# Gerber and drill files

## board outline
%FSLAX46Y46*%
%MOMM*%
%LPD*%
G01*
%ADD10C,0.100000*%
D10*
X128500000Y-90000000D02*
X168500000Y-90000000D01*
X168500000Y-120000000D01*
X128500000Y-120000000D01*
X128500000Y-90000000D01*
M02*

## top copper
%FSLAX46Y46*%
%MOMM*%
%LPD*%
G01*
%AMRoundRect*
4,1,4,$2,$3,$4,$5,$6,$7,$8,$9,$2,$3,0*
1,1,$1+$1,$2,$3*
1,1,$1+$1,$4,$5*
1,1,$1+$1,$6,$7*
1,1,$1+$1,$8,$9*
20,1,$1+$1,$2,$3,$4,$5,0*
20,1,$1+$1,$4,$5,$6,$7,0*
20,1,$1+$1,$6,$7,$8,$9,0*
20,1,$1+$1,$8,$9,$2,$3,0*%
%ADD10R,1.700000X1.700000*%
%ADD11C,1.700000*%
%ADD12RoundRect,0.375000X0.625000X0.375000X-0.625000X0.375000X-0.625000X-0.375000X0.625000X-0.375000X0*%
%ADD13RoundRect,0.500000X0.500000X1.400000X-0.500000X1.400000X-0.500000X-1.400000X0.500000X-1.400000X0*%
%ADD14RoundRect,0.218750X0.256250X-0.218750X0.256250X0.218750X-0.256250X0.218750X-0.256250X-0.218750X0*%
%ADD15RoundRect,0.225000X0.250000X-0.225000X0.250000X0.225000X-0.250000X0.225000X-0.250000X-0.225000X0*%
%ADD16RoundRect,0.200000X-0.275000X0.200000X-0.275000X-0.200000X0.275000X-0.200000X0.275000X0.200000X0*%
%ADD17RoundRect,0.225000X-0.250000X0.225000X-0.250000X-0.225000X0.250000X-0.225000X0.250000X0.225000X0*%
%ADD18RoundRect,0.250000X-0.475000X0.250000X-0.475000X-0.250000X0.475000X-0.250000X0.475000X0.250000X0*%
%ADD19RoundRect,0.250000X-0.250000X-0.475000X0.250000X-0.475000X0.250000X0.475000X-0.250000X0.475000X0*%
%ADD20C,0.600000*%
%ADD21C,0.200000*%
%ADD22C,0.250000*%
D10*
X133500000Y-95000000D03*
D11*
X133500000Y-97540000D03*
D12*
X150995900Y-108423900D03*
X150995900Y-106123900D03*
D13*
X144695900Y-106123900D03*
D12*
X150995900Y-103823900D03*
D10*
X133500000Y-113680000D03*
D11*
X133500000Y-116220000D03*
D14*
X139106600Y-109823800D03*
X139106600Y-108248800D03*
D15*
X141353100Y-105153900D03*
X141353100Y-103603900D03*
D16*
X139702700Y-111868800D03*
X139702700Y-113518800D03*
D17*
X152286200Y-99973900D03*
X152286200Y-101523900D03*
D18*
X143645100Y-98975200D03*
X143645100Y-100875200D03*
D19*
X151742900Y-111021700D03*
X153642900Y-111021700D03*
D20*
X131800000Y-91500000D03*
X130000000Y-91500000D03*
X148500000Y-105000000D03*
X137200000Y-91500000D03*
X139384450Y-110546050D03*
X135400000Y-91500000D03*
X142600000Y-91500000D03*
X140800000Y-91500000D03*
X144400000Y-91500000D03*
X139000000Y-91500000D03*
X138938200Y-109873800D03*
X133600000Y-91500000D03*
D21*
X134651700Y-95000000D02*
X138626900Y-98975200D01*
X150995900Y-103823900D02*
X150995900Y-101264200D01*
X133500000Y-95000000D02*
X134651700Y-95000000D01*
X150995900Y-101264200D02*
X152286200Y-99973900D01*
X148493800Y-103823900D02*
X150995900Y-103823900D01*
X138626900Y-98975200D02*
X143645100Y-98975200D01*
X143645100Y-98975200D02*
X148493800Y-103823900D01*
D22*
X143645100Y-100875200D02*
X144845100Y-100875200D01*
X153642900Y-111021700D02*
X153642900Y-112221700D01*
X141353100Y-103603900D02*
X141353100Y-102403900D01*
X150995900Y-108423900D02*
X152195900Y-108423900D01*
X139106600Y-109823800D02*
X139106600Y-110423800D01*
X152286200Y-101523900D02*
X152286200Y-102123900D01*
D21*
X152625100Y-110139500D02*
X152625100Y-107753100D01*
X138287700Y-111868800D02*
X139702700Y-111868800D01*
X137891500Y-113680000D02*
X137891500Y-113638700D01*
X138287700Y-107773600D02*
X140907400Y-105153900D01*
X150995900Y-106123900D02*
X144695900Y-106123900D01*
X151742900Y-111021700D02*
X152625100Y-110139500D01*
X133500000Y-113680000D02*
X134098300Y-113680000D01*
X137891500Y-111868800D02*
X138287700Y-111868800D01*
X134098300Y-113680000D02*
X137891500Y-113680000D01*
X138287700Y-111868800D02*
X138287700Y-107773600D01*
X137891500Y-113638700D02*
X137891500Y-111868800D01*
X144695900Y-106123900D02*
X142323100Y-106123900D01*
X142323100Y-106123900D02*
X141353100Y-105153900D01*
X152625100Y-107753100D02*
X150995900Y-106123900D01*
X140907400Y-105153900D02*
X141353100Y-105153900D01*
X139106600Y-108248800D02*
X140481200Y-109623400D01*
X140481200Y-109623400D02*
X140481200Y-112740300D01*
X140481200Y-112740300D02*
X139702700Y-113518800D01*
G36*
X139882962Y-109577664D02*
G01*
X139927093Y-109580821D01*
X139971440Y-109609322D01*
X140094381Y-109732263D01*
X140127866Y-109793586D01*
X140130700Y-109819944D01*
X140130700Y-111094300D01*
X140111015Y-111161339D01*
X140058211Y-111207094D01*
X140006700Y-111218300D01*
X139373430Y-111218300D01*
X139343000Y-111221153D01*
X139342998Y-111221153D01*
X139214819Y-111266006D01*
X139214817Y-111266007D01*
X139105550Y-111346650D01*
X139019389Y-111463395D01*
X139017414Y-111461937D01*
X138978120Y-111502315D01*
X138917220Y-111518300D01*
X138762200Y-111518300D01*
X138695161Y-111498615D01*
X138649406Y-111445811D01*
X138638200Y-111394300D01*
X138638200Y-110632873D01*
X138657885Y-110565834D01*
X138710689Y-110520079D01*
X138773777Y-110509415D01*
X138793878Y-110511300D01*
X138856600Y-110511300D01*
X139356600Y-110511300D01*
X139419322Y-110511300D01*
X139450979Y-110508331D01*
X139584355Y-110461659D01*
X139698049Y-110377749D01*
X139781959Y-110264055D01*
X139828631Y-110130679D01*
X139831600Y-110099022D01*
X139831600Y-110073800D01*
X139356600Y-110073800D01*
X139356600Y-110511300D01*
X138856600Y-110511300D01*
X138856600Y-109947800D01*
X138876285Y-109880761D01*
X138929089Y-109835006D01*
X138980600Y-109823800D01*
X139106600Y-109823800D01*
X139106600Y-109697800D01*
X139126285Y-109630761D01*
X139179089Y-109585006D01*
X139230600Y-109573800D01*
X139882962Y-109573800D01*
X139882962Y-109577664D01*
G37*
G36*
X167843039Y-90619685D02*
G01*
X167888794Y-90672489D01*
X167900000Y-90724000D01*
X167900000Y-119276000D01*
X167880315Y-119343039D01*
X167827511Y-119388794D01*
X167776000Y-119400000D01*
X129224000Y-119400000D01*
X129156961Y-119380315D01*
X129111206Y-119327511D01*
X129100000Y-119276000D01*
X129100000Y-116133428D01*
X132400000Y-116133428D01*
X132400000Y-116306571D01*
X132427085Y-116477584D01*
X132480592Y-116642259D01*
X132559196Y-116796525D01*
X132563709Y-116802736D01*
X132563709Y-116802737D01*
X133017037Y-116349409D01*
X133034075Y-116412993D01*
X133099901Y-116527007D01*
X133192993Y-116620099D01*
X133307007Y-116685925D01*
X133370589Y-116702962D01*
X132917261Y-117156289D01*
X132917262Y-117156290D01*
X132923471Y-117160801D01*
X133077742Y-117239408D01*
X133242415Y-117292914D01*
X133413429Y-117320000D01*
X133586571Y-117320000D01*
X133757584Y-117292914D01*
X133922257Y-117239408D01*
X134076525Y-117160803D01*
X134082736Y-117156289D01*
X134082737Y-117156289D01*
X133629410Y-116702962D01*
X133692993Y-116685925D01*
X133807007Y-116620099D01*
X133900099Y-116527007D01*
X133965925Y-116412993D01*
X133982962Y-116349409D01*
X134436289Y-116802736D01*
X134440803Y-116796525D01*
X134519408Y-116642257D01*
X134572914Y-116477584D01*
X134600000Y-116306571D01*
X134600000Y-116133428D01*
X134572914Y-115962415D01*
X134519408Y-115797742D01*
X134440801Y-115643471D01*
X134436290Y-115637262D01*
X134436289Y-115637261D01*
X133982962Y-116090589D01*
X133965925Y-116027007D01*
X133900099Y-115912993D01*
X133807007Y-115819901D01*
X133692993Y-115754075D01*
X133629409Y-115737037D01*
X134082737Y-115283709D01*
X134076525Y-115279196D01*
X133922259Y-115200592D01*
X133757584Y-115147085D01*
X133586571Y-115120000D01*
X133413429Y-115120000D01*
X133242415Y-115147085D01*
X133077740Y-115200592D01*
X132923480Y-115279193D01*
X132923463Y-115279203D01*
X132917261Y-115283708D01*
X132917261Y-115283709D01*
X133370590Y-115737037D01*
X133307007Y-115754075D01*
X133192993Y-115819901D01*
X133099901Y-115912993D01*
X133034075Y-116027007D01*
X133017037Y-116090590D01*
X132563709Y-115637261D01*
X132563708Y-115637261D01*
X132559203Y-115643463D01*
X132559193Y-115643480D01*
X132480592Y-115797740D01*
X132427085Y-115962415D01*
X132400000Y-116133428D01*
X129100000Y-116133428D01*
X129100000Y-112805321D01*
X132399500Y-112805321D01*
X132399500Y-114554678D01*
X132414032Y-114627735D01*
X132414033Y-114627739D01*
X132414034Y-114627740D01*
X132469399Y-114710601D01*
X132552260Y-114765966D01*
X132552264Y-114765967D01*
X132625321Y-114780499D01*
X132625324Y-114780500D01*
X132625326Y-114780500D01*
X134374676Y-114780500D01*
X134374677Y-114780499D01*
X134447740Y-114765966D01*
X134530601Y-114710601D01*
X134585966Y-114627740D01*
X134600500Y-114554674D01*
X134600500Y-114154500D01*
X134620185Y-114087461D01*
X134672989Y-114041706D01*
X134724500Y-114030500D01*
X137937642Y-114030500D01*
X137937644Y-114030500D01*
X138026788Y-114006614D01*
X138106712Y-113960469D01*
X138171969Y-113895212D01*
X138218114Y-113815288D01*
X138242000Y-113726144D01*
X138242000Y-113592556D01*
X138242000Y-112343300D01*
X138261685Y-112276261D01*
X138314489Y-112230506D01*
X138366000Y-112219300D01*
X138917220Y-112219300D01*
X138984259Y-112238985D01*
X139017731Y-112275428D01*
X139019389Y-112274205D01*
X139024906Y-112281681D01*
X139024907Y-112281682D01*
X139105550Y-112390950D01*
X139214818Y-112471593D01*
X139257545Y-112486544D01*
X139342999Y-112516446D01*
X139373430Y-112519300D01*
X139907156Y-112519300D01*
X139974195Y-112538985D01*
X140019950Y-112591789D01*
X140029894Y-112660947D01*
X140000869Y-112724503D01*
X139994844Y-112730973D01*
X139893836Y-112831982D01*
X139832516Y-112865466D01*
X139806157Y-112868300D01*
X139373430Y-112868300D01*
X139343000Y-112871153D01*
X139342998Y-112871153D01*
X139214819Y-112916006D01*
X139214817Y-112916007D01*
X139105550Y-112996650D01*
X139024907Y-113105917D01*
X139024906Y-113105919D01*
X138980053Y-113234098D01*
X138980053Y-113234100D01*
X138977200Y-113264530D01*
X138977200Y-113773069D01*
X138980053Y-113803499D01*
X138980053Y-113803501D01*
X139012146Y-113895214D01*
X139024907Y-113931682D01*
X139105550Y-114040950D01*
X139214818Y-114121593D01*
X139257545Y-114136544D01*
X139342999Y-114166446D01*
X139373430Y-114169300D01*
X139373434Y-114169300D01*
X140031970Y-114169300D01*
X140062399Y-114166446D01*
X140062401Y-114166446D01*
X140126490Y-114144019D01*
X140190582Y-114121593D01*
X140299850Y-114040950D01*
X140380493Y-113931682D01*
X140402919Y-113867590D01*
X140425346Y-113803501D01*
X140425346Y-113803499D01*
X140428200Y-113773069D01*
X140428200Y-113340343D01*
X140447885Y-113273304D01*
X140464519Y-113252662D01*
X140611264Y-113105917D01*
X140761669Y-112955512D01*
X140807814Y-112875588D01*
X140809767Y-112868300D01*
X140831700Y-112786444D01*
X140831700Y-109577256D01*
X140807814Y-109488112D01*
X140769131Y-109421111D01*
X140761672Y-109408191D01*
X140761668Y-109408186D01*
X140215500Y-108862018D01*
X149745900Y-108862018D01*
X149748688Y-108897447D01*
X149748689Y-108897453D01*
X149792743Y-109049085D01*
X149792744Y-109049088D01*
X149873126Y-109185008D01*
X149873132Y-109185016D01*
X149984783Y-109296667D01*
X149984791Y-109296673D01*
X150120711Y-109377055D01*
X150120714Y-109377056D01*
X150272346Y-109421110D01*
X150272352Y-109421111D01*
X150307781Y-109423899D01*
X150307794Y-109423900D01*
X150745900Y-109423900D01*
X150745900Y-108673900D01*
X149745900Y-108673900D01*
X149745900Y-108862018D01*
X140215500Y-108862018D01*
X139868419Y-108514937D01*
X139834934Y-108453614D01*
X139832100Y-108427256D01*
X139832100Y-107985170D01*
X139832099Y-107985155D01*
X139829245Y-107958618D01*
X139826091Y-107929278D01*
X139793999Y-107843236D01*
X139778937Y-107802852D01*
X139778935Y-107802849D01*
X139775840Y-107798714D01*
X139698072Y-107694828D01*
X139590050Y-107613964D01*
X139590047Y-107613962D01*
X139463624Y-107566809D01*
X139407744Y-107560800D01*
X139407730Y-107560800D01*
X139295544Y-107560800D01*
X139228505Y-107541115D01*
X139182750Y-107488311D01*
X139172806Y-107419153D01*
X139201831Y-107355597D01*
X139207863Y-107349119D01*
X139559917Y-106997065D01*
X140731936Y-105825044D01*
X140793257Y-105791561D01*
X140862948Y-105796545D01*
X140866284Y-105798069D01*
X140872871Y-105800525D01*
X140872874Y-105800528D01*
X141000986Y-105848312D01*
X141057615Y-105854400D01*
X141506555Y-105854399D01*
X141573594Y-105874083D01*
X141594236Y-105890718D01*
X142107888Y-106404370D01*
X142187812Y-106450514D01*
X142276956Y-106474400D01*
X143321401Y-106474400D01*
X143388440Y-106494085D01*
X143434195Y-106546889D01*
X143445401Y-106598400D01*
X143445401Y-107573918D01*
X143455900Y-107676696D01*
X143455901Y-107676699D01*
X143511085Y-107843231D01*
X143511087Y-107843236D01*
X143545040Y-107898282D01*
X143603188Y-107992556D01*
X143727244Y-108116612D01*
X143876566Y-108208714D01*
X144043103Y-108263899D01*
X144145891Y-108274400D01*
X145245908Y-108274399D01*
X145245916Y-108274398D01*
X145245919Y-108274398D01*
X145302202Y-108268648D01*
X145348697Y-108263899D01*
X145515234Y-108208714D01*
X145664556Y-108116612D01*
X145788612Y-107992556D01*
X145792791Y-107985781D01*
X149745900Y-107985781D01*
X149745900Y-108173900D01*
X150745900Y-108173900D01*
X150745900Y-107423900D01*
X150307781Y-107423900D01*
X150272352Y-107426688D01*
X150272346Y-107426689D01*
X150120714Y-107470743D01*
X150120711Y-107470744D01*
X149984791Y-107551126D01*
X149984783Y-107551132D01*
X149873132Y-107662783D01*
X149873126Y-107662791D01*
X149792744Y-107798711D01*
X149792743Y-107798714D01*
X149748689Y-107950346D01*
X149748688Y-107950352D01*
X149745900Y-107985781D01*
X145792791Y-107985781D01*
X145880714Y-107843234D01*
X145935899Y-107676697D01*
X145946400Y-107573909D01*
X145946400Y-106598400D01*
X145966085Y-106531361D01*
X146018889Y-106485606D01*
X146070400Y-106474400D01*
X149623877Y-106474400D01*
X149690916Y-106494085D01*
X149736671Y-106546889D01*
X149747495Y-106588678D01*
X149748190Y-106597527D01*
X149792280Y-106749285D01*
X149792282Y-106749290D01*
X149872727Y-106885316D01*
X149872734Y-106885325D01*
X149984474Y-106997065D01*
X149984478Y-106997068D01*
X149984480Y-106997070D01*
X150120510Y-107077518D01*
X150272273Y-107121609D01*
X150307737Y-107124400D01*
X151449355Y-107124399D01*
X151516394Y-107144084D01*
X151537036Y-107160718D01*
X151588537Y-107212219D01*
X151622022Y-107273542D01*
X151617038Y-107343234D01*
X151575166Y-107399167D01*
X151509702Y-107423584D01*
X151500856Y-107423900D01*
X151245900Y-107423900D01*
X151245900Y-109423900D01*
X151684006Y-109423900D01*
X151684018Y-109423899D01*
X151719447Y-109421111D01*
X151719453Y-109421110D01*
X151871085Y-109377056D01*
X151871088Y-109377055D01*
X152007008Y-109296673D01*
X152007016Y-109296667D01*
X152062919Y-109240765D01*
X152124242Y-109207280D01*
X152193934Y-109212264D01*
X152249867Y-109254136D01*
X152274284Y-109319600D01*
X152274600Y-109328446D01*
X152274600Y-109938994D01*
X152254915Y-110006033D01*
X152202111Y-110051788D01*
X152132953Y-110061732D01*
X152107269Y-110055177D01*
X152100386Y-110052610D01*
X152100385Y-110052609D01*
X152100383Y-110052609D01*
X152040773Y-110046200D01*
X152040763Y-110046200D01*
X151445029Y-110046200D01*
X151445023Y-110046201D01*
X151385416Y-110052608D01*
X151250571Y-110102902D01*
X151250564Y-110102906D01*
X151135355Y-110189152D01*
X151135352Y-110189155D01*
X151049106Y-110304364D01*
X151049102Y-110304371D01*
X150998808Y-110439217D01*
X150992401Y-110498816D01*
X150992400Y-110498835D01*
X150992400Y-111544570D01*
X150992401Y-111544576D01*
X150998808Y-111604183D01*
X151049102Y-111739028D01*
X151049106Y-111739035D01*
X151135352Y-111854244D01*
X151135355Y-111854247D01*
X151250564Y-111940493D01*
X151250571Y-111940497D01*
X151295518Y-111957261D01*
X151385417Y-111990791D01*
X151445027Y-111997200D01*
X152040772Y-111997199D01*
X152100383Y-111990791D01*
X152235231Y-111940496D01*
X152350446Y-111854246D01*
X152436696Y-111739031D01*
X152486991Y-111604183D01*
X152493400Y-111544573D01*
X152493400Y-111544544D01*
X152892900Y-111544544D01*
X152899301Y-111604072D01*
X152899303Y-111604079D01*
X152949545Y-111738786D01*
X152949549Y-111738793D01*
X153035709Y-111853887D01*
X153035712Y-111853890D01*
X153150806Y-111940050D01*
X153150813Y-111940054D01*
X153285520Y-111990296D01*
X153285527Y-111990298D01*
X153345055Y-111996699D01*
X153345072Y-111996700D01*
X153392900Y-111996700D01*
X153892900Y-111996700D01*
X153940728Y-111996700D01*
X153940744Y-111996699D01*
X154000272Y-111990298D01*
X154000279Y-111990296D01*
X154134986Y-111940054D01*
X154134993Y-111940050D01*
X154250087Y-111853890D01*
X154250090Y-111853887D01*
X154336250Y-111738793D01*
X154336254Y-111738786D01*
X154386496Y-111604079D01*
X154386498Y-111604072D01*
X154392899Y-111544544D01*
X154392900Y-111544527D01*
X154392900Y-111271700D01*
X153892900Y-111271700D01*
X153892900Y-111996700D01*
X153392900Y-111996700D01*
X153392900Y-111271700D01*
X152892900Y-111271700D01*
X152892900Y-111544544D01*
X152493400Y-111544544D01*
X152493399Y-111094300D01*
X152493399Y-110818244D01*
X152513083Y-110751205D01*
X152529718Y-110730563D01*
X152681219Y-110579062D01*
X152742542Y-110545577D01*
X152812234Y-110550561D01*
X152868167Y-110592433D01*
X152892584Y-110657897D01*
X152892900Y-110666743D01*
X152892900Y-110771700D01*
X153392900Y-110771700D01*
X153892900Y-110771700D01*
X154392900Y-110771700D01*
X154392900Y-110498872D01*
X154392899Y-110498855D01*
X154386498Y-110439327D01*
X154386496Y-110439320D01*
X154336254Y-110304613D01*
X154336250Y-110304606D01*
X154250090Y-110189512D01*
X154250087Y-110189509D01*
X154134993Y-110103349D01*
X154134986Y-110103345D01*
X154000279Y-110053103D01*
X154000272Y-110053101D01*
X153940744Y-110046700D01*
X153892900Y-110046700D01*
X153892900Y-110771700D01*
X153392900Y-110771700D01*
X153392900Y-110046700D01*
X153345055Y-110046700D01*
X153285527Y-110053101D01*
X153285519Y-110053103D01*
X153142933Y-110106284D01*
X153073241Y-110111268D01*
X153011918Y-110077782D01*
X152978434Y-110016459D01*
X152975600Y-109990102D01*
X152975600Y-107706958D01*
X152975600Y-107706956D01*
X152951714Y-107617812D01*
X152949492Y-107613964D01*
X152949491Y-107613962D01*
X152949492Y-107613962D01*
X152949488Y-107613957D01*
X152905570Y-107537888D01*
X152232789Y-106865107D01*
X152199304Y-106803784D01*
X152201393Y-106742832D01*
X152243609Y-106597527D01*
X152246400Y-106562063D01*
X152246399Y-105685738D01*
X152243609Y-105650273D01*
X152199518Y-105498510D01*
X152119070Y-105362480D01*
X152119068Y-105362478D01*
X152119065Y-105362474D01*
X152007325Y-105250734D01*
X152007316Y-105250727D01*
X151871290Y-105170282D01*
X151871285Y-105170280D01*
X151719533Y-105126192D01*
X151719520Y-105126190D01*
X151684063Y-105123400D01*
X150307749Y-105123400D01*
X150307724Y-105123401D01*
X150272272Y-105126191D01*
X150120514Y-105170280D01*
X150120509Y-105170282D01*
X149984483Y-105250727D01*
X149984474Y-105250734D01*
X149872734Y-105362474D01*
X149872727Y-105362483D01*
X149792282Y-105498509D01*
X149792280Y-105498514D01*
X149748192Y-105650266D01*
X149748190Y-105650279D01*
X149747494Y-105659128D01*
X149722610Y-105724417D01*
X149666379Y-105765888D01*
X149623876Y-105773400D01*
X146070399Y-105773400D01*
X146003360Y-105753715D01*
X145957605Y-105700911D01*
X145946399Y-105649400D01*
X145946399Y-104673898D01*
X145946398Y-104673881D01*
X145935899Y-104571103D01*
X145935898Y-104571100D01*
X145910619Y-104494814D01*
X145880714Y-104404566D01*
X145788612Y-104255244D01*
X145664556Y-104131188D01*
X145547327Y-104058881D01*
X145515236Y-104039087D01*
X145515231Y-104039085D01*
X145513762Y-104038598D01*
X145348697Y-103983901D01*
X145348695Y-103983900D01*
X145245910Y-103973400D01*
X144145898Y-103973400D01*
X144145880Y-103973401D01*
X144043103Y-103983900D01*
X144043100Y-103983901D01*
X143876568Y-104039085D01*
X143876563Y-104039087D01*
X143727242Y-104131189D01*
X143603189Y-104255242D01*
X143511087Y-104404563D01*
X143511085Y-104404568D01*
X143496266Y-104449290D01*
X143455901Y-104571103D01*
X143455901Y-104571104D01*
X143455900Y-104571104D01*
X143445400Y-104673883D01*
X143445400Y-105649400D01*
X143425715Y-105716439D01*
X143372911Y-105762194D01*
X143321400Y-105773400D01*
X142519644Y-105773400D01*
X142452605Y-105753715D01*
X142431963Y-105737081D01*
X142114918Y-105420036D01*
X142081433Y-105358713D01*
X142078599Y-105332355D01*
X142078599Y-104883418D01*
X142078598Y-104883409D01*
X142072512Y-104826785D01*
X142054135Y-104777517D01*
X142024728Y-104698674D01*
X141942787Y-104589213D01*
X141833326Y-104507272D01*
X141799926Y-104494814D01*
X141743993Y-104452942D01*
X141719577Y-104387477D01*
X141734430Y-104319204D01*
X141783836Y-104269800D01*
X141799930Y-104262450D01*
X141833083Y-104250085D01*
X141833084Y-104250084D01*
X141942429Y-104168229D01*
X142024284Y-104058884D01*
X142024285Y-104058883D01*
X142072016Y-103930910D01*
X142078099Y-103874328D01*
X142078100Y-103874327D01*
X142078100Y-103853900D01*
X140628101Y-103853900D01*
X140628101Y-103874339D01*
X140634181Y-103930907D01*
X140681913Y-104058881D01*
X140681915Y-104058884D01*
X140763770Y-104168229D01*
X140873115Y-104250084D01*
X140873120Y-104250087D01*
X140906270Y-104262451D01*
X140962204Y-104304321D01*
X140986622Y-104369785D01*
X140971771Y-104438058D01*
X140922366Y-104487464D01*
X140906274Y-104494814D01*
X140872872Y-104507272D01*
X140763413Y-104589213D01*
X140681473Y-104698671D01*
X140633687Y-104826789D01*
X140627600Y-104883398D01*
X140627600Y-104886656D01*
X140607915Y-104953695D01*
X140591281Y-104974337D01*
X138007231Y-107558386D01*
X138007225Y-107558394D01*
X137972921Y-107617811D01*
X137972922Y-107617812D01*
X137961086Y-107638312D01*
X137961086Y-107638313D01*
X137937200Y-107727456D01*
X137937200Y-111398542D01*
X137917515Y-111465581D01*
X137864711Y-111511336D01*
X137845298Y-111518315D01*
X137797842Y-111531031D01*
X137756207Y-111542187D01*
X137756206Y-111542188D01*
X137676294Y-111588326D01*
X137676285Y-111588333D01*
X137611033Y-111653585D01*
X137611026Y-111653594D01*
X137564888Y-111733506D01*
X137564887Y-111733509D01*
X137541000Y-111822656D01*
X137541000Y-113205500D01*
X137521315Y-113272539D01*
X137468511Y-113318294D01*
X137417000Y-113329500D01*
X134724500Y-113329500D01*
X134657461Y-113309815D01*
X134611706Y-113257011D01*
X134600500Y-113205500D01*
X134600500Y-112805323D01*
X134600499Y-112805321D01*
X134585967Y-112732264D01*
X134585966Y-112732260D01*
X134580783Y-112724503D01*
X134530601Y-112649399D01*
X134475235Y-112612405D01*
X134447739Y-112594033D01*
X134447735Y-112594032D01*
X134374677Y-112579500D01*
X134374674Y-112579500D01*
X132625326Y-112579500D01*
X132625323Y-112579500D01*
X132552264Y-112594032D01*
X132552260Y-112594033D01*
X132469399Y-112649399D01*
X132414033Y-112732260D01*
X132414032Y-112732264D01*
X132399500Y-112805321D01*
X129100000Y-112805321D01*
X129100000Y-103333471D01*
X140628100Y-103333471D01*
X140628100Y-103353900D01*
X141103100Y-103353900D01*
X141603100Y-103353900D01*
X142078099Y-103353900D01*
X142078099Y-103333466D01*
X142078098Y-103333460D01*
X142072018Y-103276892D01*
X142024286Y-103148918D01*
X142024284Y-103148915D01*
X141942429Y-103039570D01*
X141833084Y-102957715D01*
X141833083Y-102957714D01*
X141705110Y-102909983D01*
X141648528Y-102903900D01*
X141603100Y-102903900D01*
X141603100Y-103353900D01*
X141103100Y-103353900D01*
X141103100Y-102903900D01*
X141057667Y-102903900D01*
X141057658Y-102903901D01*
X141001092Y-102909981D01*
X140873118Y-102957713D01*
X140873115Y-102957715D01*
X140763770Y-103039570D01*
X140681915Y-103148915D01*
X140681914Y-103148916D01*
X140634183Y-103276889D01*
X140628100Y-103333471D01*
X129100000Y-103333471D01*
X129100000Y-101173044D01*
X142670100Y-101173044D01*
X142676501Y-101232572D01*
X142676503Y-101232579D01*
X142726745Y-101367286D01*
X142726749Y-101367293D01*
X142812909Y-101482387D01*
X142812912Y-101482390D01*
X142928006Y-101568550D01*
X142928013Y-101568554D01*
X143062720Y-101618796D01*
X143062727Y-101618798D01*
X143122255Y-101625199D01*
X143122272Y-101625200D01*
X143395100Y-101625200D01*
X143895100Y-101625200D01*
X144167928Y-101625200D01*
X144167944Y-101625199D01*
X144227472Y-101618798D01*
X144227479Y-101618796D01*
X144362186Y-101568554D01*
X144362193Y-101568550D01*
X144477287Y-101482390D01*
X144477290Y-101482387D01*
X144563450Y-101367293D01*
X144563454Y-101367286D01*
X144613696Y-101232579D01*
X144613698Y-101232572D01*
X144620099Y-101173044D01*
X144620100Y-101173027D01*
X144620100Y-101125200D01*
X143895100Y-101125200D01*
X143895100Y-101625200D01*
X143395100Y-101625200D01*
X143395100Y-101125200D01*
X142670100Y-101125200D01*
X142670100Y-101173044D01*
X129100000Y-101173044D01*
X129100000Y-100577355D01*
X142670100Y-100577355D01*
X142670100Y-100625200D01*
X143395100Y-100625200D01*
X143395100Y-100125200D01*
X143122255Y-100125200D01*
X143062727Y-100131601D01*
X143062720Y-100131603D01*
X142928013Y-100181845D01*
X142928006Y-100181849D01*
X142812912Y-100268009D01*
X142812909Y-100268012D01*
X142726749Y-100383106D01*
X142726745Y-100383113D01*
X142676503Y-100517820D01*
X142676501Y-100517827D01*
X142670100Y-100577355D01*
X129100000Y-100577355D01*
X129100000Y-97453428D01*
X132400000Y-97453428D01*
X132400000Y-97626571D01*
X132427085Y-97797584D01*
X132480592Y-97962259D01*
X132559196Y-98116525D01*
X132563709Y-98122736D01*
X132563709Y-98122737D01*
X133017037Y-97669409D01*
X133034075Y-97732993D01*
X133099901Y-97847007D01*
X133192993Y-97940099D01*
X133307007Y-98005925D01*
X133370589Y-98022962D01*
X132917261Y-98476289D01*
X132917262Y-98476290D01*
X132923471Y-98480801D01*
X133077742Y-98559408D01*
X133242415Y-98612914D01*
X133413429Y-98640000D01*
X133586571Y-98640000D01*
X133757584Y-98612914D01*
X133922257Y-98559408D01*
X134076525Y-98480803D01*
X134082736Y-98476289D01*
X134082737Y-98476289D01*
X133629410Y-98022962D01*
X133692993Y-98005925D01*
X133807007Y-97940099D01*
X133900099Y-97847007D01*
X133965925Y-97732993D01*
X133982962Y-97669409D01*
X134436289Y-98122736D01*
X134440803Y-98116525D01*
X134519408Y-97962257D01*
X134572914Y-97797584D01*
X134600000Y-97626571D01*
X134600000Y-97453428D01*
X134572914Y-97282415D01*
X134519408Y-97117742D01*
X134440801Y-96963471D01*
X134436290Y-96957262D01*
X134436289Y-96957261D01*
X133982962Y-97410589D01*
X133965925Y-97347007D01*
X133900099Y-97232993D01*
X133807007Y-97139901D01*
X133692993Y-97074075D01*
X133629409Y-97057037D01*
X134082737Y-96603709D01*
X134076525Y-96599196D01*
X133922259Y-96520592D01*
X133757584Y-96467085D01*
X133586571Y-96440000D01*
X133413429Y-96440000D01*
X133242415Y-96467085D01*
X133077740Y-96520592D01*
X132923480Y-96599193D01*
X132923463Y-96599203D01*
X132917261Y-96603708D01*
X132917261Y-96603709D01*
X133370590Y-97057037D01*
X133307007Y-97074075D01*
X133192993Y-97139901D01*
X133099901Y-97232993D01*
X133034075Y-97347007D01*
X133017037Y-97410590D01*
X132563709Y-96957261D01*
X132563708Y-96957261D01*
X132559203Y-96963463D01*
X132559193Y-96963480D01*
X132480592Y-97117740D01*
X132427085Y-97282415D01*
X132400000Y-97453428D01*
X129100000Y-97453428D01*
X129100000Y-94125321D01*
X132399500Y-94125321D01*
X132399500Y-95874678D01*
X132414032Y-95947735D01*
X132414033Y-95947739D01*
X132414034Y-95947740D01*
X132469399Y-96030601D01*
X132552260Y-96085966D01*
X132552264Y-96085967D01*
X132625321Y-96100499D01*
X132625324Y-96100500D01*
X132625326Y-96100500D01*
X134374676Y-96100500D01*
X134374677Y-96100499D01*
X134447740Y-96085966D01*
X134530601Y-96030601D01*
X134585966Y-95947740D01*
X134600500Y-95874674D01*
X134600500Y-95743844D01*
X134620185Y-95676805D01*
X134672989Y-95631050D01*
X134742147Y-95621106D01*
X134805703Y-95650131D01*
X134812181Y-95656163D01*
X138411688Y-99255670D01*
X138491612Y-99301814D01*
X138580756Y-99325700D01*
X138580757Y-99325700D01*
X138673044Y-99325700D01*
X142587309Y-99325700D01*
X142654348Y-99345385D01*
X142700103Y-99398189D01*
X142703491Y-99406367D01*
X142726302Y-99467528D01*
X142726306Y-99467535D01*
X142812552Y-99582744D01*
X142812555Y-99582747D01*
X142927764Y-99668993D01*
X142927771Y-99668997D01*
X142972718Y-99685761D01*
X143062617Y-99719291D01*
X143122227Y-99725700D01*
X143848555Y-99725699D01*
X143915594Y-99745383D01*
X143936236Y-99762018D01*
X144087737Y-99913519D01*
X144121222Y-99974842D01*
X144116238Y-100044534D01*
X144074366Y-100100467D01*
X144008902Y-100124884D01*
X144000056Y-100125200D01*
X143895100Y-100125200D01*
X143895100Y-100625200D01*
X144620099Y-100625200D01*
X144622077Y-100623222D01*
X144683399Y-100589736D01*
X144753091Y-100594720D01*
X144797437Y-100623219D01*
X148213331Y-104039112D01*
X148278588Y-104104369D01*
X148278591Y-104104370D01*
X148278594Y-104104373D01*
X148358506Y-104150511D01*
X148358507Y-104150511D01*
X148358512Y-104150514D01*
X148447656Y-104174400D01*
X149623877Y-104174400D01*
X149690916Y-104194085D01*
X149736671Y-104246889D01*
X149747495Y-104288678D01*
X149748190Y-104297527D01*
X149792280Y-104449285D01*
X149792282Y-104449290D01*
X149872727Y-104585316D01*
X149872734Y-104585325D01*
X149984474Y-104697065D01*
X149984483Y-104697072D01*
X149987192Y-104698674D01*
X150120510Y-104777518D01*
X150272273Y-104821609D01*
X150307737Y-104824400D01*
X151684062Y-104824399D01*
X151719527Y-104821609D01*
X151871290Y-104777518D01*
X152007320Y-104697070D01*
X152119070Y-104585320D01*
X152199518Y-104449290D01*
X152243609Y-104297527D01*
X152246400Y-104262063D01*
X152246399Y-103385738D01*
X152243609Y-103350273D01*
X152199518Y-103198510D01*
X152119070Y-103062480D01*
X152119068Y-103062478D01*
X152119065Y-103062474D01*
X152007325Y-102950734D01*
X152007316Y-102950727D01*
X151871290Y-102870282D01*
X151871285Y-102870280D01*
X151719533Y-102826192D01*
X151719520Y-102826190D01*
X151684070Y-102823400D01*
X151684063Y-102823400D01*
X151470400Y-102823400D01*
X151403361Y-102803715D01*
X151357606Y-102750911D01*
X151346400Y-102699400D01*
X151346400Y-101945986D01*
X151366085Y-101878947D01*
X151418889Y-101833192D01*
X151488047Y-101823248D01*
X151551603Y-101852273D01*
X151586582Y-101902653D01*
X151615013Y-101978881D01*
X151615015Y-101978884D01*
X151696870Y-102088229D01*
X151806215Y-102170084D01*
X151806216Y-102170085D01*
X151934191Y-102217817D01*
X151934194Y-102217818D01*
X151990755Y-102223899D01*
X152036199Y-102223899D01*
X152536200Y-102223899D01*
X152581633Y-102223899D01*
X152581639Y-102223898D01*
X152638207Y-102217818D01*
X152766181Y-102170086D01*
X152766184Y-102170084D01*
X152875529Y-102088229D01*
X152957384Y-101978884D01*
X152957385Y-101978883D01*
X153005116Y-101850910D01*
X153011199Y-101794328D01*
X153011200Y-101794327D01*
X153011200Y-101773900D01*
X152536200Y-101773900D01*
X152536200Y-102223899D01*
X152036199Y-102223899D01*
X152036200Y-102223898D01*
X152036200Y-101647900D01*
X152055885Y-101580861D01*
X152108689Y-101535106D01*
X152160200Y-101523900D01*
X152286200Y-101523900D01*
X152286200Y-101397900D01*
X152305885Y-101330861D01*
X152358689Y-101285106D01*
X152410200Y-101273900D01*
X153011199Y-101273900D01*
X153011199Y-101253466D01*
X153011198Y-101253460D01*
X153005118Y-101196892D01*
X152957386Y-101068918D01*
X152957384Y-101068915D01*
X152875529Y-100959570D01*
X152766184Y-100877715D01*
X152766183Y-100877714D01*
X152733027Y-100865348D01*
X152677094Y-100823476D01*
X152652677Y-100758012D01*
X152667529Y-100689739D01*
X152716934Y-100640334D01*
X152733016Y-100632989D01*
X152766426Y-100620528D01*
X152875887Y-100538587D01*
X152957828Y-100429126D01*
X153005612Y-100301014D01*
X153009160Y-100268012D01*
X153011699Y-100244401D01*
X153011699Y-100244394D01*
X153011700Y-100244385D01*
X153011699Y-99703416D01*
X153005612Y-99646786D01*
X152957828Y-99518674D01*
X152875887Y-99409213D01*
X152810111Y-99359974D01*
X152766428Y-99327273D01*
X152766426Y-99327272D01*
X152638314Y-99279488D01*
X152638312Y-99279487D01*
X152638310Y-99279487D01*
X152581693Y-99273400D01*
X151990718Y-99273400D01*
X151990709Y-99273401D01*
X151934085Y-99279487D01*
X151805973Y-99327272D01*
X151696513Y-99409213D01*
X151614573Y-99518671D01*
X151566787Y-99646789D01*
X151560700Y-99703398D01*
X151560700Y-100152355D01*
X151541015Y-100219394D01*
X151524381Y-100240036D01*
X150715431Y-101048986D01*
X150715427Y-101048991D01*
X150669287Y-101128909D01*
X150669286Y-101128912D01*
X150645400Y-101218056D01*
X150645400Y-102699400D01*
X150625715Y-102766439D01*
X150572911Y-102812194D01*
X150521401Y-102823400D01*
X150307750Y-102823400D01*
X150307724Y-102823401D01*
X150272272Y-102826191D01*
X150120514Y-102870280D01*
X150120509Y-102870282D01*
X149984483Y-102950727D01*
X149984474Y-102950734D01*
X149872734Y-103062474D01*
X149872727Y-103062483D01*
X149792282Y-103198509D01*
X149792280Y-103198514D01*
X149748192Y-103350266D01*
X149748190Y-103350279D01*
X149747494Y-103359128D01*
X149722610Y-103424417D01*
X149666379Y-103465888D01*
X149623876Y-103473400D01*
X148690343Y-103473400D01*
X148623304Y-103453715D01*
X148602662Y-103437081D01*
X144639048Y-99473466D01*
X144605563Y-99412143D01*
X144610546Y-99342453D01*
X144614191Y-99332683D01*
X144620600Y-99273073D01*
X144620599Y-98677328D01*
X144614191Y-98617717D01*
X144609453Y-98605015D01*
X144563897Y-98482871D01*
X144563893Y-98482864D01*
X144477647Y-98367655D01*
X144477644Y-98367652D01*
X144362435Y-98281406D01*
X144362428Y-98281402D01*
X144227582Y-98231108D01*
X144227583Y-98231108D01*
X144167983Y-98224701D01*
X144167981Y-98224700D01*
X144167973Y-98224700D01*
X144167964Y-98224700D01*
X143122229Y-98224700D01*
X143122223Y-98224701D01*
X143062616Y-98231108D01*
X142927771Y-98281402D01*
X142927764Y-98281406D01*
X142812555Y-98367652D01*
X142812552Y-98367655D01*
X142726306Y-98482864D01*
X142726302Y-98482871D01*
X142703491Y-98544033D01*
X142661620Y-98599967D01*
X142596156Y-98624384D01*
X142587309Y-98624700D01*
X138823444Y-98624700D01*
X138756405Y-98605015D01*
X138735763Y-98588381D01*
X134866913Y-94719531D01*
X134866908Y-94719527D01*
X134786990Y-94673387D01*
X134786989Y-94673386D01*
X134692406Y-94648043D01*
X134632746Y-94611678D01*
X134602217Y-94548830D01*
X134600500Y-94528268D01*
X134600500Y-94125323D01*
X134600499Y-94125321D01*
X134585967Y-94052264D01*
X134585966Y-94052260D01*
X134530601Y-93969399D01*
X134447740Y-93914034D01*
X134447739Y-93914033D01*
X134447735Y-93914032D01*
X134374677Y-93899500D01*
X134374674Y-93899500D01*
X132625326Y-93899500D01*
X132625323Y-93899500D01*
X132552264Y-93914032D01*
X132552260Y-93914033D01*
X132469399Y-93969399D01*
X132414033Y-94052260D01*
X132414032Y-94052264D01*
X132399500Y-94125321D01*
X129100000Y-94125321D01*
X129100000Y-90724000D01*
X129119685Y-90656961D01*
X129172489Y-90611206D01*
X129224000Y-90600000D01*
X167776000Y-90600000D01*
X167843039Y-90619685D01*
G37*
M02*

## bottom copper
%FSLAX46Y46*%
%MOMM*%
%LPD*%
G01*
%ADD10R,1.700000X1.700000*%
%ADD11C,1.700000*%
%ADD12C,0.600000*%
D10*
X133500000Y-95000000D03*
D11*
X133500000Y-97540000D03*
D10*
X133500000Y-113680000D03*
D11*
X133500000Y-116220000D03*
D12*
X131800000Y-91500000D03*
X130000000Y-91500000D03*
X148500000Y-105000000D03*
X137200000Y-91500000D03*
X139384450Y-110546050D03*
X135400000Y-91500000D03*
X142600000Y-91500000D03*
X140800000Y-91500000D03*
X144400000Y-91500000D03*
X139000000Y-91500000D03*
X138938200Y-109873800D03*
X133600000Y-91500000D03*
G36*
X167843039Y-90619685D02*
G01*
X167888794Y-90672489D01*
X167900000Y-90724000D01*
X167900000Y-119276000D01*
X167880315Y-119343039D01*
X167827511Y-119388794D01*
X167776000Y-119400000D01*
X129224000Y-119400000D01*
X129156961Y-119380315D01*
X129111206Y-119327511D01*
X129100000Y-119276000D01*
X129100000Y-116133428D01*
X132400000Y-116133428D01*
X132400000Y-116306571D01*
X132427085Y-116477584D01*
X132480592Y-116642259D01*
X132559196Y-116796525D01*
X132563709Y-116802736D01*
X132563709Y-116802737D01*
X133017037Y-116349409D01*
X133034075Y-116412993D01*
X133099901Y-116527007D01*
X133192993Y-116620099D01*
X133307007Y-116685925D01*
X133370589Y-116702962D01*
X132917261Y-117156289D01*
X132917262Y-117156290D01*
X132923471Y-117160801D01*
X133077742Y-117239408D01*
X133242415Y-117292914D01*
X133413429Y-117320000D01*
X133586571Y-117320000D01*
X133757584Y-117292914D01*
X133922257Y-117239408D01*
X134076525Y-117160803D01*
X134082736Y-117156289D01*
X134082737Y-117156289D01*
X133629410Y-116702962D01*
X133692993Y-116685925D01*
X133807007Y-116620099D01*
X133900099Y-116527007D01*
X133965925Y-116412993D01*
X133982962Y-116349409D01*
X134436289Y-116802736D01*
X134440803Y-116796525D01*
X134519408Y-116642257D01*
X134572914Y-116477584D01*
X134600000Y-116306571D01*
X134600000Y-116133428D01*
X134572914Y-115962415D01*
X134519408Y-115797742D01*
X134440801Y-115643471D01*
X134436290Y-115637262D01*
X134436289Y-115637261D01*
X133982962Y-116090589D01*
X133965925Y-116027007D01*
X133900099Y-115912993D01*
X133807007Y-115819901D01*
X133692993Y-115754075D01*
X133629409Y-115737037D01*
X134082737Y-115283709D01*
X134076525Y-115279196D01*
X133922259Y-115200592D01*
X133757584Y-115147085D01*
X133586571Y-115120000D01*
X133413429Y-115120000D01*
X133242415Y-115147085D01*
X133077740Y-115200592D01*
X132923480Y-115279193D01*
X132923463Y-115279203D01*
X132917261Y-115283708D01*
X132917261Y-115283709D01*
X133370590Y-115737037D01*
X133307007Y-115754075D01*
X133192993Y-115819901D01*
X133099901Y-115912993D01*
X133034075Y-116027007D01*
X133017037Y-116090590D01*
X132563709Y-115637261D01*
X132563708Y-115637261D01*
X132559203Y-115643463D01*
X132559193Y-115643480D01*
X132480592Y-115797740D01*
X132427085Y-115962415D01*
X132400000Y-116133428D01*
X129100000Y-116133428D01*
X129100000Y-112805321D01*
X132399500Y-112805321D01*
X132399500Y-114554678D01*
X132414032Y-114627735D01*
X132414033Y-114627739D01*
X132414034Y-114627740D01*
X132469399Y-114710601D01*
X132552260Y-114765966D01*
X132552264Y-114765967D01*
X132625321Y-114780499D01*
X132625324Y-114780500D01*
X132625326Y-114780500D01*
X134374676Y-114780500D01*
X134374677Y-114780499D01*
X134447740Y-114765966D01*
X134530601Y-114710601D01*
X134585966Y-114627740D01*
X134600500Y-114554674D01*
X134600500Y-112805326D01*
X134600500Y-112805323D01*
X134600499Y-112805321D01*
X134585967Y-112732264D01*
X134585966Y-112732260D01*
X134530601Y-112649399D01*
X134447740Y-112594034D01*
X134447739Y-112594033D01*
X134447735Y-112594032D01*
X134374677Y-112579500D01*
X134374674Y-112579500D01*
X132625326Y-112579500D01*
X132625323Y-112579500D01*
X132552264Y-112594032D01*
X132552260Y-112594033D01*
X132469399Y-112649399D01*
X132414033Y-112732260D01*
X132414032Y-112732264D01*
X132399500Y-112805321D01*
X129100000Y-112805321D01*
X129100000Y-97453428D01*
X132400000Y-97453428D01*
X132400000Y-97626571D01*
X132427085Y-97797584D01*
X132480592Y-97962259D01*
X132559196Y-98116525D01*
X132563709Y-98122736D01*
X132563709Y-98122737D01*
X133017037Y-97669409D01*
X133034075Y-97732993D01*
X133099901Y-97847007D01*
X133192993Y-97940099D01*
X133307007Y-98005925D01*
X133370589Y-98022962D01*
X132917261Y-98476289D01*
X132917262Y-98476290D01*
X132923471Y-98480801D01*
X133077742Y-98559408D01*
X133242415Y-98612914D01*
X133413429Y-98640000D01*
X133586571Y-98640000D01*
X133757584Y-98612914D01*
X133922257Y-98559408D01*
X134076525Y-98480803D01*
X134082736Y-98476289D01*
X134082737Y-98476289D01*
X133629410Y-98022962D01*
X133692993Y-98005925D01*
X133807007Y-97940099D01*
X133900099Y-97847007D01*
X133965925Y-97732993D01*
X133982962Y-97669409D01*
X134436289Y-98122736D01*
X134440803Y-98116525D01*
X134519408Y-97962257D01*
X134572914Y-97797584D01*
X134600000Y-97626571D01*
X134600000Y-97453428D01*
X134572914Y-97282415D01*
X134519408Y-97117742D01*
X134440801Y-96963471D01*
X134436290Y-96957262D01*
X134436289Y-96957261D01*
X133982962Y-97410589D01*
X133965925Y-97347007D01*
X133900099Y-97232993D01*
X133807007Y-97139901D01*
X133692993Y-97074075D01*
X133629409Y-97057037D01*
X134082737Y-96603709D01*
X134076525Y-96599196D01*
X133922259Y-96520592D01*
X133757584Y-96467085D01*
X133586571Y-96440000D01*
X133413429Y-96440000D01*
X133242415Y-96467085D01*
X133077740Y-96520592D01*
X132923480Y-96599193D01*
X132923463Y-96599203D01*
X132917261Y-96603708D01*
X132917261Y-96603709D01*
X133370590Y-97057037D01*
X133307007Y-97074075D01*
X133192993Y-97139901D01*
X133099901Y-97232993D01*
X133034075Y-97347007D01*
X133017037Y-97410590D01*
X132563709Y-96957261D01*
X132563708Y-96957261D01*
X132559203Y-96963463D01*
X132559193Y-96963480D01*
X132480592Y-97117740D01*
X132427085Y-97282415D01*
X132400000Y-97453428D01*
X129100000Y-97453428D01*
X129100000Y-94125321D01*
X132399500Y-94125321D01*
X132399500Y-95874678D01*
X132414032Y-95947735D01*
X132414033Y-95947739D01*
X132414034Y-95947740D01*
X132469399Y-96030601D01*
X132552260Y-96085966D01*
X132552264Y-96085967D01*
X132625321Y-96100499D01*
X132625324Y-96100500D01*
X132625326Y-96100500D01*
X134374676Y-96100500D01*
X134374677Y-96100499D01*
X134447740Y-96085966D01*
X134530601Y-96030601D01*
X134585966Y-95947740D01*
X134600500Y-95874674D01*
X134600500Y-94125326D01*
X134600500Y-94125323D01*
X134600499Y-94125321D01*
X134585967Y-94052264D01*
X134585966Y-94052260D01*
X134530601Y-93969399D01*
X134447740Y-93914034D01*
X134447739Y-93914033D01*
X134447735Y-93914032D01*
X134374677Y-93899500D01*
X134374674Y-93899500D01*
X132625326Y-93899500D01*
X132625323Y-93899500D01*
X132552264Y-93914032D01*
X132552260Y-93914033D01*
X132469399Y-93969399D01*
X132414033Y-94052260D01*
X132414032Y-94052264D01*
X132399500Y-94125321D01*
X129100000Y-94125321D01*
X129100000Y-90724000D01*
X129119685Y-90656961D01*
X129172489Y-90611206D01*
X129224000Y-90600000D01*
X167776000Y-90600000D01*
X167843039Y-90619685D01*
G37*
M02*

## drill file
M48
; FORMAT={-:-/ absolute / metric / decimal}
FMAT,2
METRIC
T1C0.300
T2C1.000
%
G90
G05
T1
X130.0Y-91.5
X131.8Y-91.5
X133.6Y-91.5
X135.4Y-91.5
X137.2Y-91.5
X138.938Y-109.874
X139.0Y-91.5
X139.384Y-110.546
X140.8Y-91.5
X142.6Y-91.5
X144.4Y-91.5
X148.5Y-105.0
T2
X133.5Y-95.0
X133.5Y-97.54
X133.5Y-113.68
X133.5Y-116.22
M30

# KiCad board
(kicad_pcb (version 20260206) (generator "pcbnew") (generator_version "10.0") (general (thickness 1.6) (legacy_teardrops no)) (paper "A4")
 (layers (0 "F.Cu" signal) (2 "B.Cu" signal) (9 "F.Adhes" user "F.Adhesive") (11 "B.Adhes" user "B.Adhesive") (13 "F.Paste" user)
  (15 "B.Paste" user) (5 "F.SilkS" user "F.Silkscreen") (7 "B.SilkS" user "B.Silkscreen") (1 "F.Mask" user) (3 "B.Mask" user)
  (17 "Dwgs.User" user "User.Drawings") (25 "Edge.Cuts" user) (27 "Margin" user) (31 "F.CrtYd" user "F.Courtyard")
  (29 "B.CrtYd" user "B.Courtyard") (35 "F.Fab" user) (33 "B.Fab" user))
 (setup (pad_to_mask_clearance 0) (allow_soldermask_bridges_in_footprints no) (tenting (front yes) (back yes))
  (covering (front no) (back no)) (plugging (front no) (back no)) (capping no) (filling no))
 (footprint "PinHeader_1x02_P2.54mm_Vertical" (layer "F.Cu") (at 133.5 95)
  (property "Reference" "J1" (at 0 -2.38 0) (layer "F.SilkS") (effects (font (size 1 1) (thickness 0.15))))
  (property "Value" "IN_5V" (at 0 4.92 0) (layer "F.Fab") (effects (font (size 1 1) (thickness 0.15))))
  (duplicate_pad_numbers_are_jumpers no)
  (pad "1" thru_hole rect (at 0 0) (size 1.7 1.7) (drill 1) (layers "*.Cu" "*.Mask") (remove_unused_layers no) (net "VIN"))
  (pad "2" thru_hole circle (at 0 2.54) (size 1.7 1.7) (drill 1) (layers "*.Cu" "*.Mask") (remove_unused_layers no) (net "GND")))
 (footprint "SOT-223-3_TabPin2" (layer "F.Cu") (at 147.8459 106.1239 180)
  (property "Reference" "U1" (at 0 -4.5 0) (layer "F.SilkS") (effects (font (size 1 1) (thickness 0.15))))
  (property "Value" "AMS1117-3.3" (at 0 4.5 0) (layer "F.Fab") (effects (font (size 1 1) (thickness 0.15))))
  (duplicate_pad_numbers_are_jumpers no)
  (pad "1" smd roundrect (at -3.15 -2.3 180) (size 2 1.5) (layers "F.Cu" "F.Mask" "F.Paste") (roundrect_rratio 0.25) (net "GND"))
  (pad "2" smd roundrect (at -3.15 0 180) (size 2 1.5) (layers "F.Cu" "F.Mask" "F.Paste") (roundrect_rratio 0.25) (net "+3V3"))
  (pad "2" smd roundrect (at 3.15 0 180) (size 2 3.8) (layers "F.Cu" "F.Mask" "F.Paste") (roundrect_rratio 0.25) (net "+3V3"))
  (pad "3" smd roundrect (at -3.15 2.3 180) (size 2 1.5) (layers "F.Cu" "F.Mask" "F.Paste") (roundrect_rratio 0.25) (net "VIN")))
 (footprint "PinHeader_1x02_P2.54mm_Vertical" (layer "F.Cu") (at 133.5 113.68)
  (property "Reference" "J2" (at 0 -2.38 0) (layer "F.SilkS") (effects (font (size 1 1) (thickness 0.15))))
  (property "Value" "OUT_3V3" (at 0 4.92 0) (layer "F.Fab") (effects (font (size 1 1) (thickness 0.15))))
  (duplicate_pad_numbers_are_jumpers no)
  (pad "1" thru_hole rect (at 0 0) (size 1.7 1.7) (drill 1) (layers "*.Cu" "*.Mask") (remove_unused_layers no) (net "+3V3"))
  (pad "2" thru_hole circle (at 0 2.54) (size 1.7 1.7) (drill 1) (layers "*.Cu" "*.Mask") (remove_unused_layers no) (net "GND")))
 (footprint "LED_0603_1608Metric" (layer "F.Cu") (at 139.1066 109.0363 90)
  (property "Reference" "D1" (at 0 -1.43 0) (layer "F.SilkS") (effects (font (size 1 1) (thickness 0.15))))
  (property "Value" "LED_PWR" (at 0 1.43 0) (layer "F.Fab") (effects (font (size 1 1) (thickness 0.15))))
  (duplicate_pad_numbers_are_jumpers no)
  (pad "1" smd roundrect (at -0.7875 0 90) (size 0.875 0.95) (layers "F.Cu" "F.Mask" "F.Paste") (roundrect_rratio 0.25) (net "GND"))
  (pad "2" smd roundrect (at 0.7875 0 90) (size 0.875 0.95) (layers "F.Cu" "F.Mask" "F.Paste") (roundrect_rratio 0.25) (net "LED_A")))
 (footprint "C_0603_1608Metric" (layer "F.Cu") (at 141.3531 104.3789 90)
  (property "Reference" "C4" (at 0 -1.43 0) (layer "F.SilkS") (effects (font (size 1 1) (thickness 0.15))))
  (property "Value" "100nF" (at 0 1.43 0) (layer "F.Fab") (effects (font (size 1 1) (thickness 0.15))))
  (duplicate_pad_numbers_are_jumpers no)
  (pad "1" smd roundrect (at -0.775 0 90) (size 0.9 0.95) (layers "F.Cu" "F.Mask" "F.Paste") (roundrect_rratio 0.25) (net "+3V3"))
  (pad "2" smd roundrect (at 0.775 0 90) (size 0.9 0.95) (layers "F.Cu" "F.Mask" "F.Paste") (roundrect_rratio 0.25) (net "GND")))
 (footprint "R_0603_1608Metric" (layer "F.Cu") (at 139.7027 112.6938 -90)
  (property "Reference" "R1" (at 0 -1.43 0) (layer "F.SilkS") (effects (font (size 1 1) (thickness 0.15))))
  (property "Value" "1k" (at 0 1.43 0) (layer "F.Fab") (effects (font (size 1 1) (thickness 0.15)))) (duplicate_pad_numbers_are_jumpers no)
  (pad "1" smd roundrect (at -0.825 0 270) (size 0.8 0.95) (layers "F.Cu" "F.Mask" "F.Paste") (roundrect_rratio 0.25) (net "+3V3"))
  (pad "2" smd roundrect (at 0.825 0 270) (size 0.8 0.95) (layers "F.Cu" "F.Mask" "F.Paste") (roundrect_rratio 0.25) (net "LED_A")))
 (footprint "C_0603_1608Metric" (layer "F.Cu") (at 152.2862 100.7489 -90)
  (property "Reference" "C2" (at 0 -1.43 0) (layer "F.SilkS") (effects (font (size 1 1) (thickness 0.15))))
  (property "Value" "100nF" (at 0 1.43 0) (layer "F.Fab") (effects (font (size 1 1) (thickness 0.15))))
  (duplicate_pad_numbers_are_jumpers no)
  (pad "1" smd roundrect (at -0.775 0 270) (size 0.9 0.95) (layers "F.Cu" "F.Mask" "F.Paste") (roundrect_rratio 0.25) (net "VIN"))
  (pad "2" smd roundrect (at 0.775 0 270) (size 0.9 0.95) (layers "F.Cu" "F.Mask" "F.Paste") (roundrect_rratio 0.25) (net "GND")))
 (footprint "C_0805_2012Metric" (layer "F.Cu") (at 143.6451 99.9252 -90)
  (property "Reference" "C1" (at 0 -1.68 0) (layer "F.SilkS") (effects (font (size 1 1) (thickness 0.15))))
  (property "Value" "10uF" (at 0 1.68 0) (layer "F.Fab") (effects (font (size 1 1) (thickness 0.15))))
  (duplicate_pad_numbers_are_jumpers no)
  (pad "1" smd roundrect (at -0.95 0 270) (size 1 1.45) (layers "F.Cu" "F.Mask" "F.Paste") (roundrect_rratio 0.25) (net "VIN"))
  (pad "2" smd roundrect (at 0.95 0 270) (size 1 1.45) (layers "F.Cu" "F.Mask" "F.Paste") (roundrect_rratio 0.25) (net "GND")))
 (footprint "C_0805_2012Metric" (layer "F.Cu") (at 152.6929 111.0217)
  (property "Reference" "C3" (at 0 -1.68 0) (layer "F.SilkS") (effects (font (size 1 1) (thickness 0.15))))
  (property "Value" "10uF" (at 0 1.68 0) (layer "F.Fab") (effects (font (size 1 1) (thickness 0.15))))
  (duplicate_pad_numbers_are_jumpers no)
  (pad "1" smd roundrect (at -0.95 0) (size 1 1.45) (layers "F.Cu" "F.Mask" "F.Paste") (roundrect_rratio 0.25) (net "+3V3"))
  (pad "2" smd roundrect (at 0.95 0) (size 1 1.45) (layers "F.Cu" "F.Mask" "F.Paste") (roundrect_rratio 0.25) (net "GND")))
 (gr_rect (start 128.5 90) (end 168.5 120) (stroke (width 0.1) (type default)) (fill no) (layer "Edge.Cuts"))
 (segment (start 134.6517 95) (end 138.6269 98.9752) (width 0.2) (layer "F.Cu") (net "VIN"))
 (segment (start 150.9959 103.8239) (end 150.9959 101.2642) (width 0.2) (layer "F.Cu") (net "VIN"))
 (segment (start 133.5 95) (end 134.6517 95) (width 0.2) (layer "F.Cu") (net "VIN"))
 (segment (start 150.9959 101.2642) (end 152.2862 99.9739) (width 0.2) (layer "F.Cu") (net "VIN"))
 (segment (start 148.4938 103.8239) (end 150.9959 103.8239) (width 0.2) (layer "F.Cu") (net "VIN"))
 (segment (start 138.6269 98.9752) (end 143.6451 98.9752) (width 0.2) (layer "F.Cu") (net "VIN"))
 (segment (start 143.6451 98.9752) (end 148.4938 103.8239) (width 0.2) (layer "F.Cu") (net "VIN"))
 (segment (start 143.6451 100.8752) (end 144.8451 100.8752) (width 0.25) (layer "F.Cu") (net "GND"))
 (segment (start 153.6429 111.0217) (end 153.6429 112.2217) (width 0.25) (layer "F.Cu") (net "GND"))
 (segment (start 141.3531 103.6039) (end 141.3531 102.4039) (width 0.25) (layer "F.Cu") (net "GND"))
 (segment (start 150.9959 108.4239) (end 152.1959 108.4239) (width 0.25) (layer "F.Cu") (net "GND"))
 (segment (start 139.1066 109.8238) (end 139.1066 110.4238) (width 0.25) (layer "F.Cu") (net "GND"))
 (segment (start 152.2862 101.5239) (end 152.2862 102.1239) (width 0.25) (layer "F.Cu") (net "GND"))
 (via (at 131.8 91.5) (size 0.6) (drill 0.3) (layers "F.Cu" "B.Cu") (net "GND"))
 (via (at 130 91.5) (size 0.6) (drill 0.3) (layers "F.Cu" "B.Cu") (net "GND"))
 (via (at 148.5 105) (size 0.6) (drill 0.3) (layers "F.Cu" "B.Cu") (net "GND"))
 (via (at 137.2 91.5) (size 0.6) (drill 0.3) (layers "F.Cu" "B.Cu") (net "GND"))
 (via (at 139.38445 110.54605) (size 0.6) (drill 0.3) (layers "F.Cu" "B.Cu") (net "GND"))
 (via (at 135.4 91.5) (size 0.6) (drill 0.3) (layers "F.Cu" "B.Cu") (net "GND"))
 (via (at 142.6 91.5) (size 0.6) (drill 0.3) (layers "F.Cu" "B.Cu") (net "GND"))
 (via (at 140.8 91.5) (size 0.6) (drill 0.3) (layers "F.Cu" "B.Cu") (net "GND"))
 (via (at 144.4 91.5) (size 0.6) (drill 0.3) (layers "F.Cu" "B.Cu") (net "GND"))
 (via (at 139 91.5) (size 0.6) (drill 0.3) (layers "F.Cu" "B.Cu") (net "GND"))
 (via (at 138.9382 109.8738) (size 0.6) (drill 0.3) (layers "F.Cu" "B.Cu") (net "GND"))
 (via (at 133.6 91.5) (size 0.6) (drill 0.3) (layers "F.Cu" "B.Cu") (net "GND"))
 (segment (start 152.6251 110.1395) (end 152.6251 107.7531) (width 0.2) (layer "F.Cu") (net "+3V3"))
 (segment (start 138.2877 111.8688) (end 139.7027 111.8688) (width 0.2) (layer "F.Cu") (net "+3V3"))
 (segment (start 137.8915 113.68) (end 137.8915 113.6387) (width 0.2) (layer "F.Cu") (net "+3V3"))
 (segment (start 138.2877 107.7736) (end 140.9074 105.1539) (width 0.2) (layer "F.Cu") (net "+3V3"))
 (segment (start 150.9959 106.1239) (end 144.6959 106.1239) (width 0.2) (layer "F.Cu") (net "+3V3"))
 (segment (start 151.7429 111.0217) (end 152.6251 110.1395) (width 0.2) (layer "F.Cu") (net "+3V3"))
 (segment (start 133.5 113.68) (end 134.0983 113.68) (width 0.2) (layer "F.Cu") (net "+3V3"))
 (segment (start 137.8915 111.8688) (end 138.2877 111.8688) (width 0.2) (layer "F.Cu") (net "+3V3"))
 (segment (start 134.0983 113.68) (end 137.8915 113.68) (width 0.2) (layer "F.Cu") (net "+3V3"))
 (segment (start 138.2877 111.8688) (end 138.2877 107.7736) (width 0.2) (layer "F.Cu") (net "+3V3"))
 (segment (start 137.8915 113.6387) (end 137.8915 111.8688) (width 0.2) (layer "F.Cu") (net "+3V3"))
 (segment (start 144.6959 106.1239) (end 142.3231 106.1239) (width 0.2) (layer "F.Cu") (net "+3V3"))
 (segment (start 142.3231 106.1239) (end 141.3531 105.1539) (width 0.2) (layer "F.Cu") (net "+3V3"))
 (segment (start 152.6251 107.7531) (end 150.9959 106.1239) (width 0.2) (layer "F.Cu") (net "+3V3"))
 (segment (start 140.9074 105.1539) (end 141.3531 105.1539) (width 0.2) (layer "F.Cu") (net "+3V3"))
 (segment (start 139.1066 108.2488) (end 140.4812 109.6234) (width 0.2) (layer "F.Cu") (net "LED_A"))
 (segment (start 140.4812 109.6234) (end 140.4812 112.7403) (width 0.2) (layer "F.Cu") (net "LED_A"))
 (segment (start 140.4812 112.7403) (end 139.7027 113.5188) (width 0.2) (layer "F.Cu") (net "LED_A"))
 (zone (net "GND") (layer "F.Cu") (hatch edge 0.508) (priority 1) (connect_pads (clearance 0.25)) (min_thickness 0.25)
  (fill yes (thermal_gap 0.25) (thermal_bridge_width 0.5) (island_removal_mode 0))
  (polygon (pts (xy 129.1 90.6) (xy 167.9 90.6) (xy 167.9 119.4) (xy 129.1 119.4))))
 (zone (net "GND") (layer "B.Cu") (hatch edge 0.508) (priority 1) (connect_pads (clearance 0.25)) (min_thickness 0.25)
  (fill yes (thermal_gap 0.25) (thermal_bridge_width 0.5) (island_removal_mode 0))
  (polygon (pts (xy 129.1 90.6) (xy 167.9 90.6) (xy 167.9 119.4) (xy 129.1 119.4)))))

